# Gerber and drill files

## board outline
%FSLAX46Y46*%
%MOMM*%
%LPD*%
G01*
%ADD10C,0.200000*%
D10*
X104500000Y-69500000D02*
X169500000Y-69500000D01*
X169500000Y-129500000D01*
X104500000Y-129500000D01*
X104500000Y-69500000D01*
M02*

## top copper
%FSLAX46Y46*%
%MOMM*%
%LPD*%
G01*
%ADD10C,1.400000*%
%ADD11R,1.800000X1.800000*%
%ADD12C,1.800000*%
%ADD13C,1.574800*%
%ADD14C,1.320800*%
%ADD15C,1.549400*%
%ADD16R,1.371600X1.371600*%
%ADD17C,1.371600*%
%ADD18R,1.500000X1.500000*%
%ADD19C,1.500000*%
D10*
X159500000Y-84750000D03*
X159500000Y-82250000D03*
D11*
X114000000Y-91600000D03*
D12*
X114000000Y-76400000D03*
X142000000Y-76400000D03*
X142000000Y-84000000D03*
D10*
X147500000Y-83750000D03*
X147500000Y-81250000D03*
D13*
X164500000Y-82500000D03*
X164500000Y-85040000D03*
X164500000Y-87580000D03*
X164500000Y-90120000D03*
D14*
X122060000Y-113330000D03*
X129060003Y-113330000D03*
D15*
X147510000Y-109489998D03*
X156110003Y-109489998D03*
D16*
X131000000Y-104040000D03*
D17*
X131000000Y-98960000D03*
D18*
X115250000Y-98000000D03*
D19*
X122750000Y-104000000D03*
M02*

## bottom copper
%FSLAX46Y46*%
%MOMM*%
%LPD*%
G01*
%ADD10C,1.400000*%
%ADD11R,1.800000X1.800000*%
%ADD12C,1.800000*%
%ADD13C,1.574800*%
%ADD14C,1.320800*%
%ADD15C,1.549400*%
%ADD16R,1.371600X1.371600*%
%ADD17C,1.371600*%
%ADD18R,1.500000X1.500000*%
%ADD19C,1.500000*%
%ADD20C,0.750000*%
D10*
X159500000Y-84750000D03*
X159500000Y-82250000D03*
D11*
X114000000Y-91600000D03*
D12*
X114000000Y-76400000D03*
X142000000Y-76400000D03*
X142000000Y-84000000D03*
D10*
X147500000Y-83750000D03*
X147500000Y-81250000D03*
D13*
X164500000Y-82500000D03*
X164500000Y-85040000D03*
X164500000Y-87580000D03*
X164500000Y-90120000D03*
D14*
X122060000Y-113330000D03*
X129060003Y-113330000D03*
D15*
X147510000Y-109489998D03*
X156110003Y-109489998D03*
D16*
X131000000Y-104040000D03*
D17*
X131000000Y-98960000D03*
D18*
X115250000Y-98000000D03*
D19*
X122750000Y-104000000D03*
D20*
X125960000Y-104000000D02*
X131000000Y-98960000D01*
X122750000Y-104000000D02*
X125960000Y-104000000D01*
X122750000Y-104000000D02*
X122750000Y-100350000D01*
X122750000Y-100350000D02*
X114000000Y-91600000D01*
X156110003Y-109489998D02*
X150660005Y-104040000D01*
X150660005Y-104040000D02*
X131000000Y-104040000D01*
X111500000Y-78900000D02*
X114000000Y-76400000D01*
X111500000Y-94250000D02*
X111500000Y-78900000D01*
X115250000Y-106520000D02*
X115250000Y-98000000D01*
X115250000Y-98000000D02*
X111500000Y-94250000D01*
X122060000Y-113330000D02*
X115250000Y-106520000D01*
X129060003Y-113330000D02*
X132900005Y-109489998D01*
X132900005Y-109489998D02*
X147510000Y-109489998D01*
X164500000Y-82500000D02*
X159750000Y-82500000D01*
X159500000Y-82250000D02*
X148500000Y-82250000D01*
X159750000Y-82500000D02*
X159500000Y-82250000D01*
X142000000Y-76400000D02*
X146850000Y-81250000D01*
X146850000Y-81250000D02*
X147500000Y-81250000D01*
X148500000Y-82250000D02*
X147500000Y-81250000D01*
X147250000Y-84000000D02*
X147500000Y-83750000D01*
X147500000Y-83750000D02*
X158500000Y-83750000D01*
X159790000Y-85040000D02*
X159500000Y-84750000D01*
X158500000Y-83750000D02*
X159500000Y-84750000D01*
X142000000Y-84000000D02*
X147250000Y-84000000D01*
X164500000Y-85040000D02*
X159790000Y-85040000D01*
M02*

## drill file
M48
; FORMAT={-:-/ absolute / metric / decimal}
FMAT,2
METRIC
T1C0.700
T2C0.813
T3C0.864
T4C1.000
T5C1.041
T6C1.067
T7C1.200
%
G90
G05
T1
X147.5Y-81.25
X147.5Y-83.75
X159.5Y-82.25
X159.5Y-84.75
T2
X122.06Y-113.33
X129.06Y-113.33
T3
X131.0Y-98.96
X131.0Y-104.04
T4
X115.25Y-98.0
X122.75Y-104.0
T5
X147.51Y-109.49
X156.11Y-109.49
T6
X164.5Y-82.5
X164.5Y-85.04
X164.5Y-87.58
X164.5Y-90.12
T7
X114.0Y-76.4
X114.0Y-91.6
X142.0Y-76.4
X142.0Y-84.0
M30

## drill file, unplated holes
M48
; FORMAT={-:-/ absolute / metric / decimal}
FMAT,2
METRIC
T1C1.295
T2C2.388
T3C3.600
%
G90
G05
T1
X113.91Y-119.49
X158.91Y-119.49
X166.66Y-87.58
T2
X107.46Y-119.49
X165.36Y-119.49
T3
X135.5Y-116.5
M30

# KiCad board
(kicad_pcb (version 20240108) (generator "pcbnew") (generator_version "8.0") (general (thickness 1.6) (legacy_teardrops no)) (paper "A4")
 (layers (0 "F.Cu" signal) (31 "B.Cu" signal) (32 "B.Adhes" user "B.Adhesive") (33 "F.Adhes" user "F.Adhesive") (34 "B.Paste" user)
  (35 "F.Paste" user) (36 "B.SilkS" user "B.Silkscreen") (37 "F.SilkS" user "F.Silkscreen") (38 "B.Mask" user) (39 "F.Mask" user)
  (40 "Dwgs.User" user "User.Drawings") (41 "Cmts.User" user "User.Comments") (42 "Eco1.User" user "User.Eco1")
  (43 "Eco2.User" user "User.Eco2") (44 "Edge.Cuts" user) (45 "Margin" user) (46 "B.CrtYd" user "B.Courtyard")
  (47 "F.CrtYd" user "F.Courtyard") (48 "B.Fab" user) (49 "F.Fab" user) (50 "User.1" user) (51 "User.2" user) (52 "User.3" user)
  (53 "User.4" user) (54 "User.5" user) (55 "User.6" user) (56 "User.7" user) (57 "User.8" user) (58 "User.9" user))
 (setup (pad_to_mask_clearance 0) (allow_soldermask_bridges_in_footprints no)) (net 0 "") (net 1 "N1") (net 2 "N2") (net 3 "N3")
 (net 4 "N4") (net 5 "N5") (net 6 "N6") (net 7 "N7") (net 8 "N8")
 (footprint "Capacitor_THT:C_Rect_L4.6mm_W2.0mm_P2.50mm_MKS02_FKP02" (layer "F.Cu") (at 159.5 84.75 90)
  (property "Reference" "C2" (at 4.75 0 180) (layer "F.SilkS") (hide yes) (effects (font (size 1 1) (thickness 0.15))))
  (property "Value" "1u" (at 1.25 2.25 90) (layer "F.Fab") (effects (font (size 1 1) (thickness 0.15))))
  (pad "1" thru_hole circle (at 0 0 90) (size 1.4 1.4) (drill 0.7) (layers "*.Cu" "*.Mask") (remove_unused_layers no) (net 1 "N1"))
  (pad "2" thru_hole circle (at 2.5 0 90) (size 1.4 1.4) (drill 0.7) (layers "*.Cu" "*.Mask") (remove_unused_layers no) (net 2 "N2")))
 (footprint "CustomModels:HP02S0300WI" (layer "F.Cu") (at 114 91.6)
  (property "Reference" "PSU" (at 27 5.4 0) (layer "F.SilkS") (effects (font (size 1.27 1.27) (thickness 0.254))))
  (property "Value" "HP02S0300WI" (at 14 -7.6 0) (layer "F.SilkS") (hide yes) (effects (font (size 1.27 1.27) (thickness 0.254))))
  (pad "1" thru_hole rect (at 0 0) (size 1.8 1.8) (drill 1.2) (layers "*.Cu" "*.Mask") (remove_unused_layers no) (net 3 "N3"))
  (pad "2" thru_hole circle (at 0 -15.2) (size 1.8 1.8) (drill 1.2) (layers "*.Cu" "*.Mask") (remove_unused_layers no) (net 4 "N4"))
  (pad "3" thru_hole circle (at 28 -15.2) (size 1.8 1.8) (drill 1.2) (layers "*.Cu" "*.Mask") (remove_unused_layers no) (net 2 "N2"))
  (pad "4" thru_hole circle (at 28 -7.6) (size 1.8 1.8) (drill 1.2) (layers "*.Cu" "*.Mask") (remove_unused_layers no) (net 1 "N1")))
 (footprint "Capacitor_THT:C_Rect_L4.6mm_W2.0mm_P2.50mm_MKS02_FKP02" (layer "F.Cu") (at 147.5 83.75 90)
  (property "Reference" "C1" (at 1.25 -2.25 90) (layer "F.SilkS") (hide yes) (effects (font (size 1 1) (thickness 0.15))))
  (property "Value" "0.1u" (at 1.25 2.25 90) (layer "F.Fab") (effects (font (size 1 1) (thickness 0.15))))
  (pad "1" thru_hole circle (at 0 0 90) (size 1.4 1.4) (drill 0.7) (layers "*.Cu" "*.Mask") (remove_unused_layers no) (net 1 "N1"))
  (pad "2" thru_hole circle (at 2.5 0 90) (size 1.4 1.4) (drill 0.7) (layers "*.Cu" "*.Mask") (remove_unused_layers no) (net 2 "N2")))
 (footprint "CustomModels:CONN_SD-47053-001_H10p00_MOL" (layer "F.Cu") (at 164.5 82.5 90)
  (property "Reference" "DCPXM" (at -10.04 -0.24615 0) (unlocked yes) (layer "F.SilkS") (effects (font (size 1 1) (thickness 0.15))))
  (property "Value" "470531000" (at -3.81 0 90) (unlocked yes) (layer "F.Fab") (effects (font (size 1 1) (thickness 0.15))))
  (pad "" np_thru_hole circle (at -5.08 2.16 90) (size 1.2954 1.2954) (drill 1.2954) (layers "*.SilkS"))
  (pad "1" thru_hole circle (at 0 0 90) (size 1.5748 1.5748) (drill 1.0668) (layers "*.Cu" "*.Mask") (remove_unused_layers no) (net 2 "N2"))
  (pad "2" thru_hole circle (at -2.54 0 90) (size 1.5748 1.5748) (drill 1.0668) (layers "*.Cu" "*.Mask") (remove_unused_layers no)
   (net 1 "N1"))
  (pad "3" thru_hole circle (at -5.08 0 90) (size 1.5748 1.5748) (drill 1.0668) (layers "*.Cu" "*.Mask") (remove_unused_layers no)
   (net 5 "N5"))
  (pad "4" thru_hole circle (at -7.62 0 90) (size 1.5748 1.5748) (drill 1.0668) (layers "*.Cu" "*.Mask") (remove_unused_layers no)
   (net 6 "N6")))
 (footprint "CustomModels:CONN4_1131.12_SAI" (layer "F.Cu") (at 122.06 113.33)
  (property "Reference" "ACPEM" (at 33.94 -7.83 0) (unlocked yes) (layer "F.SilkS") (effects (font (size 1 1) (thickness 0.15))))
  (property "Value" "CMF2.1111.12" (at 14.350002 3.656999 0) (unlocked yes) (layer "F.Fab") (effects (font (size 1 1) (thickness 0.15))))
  (pad "" np_thru_hole circle (at -14.600004 6.159999 90) (size 2.8956 2.8956) (drill 2.3876) (layers "*.SilkS"))
  (pad "" np_thru_hole circle (at -8.150004 6.159999 90) (size 1.8034 1.8034) (drill 1.2954) (layers "*.SilkS"))
  (pad "" np_thru_hole circle (at 13.44 3.17) (size 4.6 4.6) (drill 3.6) (layers "*.SilkS"))
  (pad "" np_thru_hole circle (at 36.850007 6.159999 90) (size 1.8034 1.8034) (drill 1.2954) (layers "*.SilkS"))
  (pad "" np_thru_hole circle (at 43.300007 6.159999 90) (size 2.8956 2.8956) (drill 2.3876) (layers "*.SilkS"))
  (pad "1" thru_hole circle (at 0 0) (size 1.3208 1.3208) (drill 0.8128) (layers "*.Cu" "*.Mask") (remove_unused_layers no) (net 4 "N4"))
  (pad "2" thru_hole circle (at 7.000003 0) (size 1.3208 1.3208) (drill 0.8128) (layers "*.Cu" "*.Mask") (remove_unused_layers no)
   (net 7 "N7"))
  (pad "3" thru_hole circle (at 25.45 -3.840002) (size 1.5494 1.5494) (drill 1.0414) (layers "*.Cu" "*.Mask") (remove_unused_layers no)
   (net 7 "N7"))
  (pad "4" thru_hole circle (at 34.050003 -3.840002) (size 1.5494 1.5494) (drill 1.0414) (layers "*.Cu" "*.Mask") (remove_unused_layers no)
   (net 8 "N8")))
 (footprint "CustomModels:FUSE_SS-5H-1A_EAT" (layer "F.Cu") (at 131 104.04 90)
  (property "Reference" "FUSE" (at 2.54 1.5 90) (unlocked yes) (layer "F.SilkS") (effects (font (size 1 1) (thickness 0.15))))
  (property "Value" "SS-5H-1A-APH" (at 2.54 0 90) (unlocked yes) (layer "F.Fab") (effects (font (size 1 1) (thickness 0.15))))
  (pad "1" thru_hole rect (at 0 0 90) (size 1.3716 1.3716) (drill 0.8636) (layers "*.Cu" "*.Mask") (remove_unused_layers no) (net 8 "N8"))
  (pad "2" thru_hole circle (at 5.08 0 90) (size 1.3716 1.3716) (drill 0.8636) (layers "*.Cu" "*.Mask") (remove_unused_layers no)
   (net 3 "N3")))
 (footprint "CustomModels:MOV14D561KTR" (layer "F.Cu") (at 115.25 98)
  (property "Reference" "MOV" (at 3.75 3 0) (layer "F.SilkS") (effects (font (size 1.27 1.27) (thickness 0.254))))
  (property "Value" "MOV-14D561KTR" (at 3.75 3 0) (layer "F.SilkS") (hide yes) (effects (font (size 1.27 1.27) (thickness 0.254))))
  (pad "1" thru_hole rect (at 0 0) (size 1.5 1.5) (drill 1) (layers "*.Cu" "*.Mask") (remove_unused_layers no) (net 4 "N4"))
  (pad "2" thru_hole circle (at 7.5 6) (size 1.5 1.5) (drill 1) (layers "*.Cu" "*.Mask") (remove_unused_layers no) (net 3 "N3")))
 (gr_rect (start 104.5 69.5) (end 169.5 129.5) (stroke (width 0.2) (type default)) (fill none) (layer "Edge.Cuts"))
 (segment (start 125.96 104) (end 131 98.96) (width 0.75) (layer "B.Cu") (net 3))
 (segment (start 122.75 104) (end 125.96 104) (width 0.75) (layer "B.Cu") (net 3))
 (segment (start 122.75 104) (end 122.75 100.35) (width 0.75) (layer "B.Cu") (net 3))
 (segment (start 122.75 100.35) (end 114 91.6) (width 0.75) (layer "B.Cu") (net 3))
 (segment (start 156.110003 109.489998) (end 150.660005 104.04) (width 0.75) (layer "B.Cu") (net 8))
 (segment (start 150.660005 104.04) (end 131 104.04) (width 0.75) (layer "B.Cu") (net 8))
 (segment (start 111.5 78.9) (end 114 76.4) (width 0.75) (layer "B.Cu") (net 4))
 (segment (start 111.5 94.25) (end 111.5 78.9) (width 0.75) (layer "B.Cu") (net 4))
 (segment (start 115.25 106.52) (end 115.25 98) (width 0.75) (layer "B.Cu") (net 4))
 (segment (start 115.25 98) (end 111.5 94.25) (width 0.75) (layer "B.Cu") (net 4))
 (segment (start 122.06 113.33) (end 115.25 106.52) (width 0.75) (layer "B.Cu") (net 4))
 (segment (start 129.060003 113.33) (end 132.900005 109.489998) (width 0.75) (layer "B.Cu") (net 7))
 (segment (start 132.900005 109.489998) (end 147.51 109.489998) (width 0.75) (layer "B.Cu") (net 7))
 (segment (start 164.5 82.5) (end 159.75 82.5) (width 0.75) (layer "B.Cu") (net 2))
 (segment (start 159.5 82.25) (end 148.5 82.25) (width 0.75) (layer "B.Cu") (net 2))
 (segment (start 159.75 82.5) (end 159.5 82.25) (width 0.75) (layer "B.Cu") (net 2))
 (segment (start 142 76.4) (end 146.85 81.25) (width 0.75) (layer "B.Cu") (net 2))
 (segment (start 146.85 81.25) (end 147.5 81.25) (width 0.75) (layer "B.Cu") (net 2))
 (segment (start 148.5 82.25) (end 147.5 81.25) (width 0.75) (layer "B.Cu") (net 2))
 (segment (start 147.25 84) (end 147.5 83.75) (width 0.75) (layer "B.Cu") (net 1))
 (segment (start 147.5 83.75) (end 158.5 83.75) (width 0.75) (layer "B.Cu") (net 1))
 (segment (start 159.79 85.04) (end 159.5 84.75) (width 0.75) (layer "B.Cu") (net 1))
 (segment (start 158.5 83.75) (end 159.5 84.75) (width 0.75) (layer "B.Cu") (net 1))
 (segment (start 142 84) (end 147.25 84) (width 0.75) (layer "B.Cu") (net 1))
 (segment (start 164.5 85.04) (end 159.79 85.04) (width 0.75) (layer "B.Cu") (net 1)))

